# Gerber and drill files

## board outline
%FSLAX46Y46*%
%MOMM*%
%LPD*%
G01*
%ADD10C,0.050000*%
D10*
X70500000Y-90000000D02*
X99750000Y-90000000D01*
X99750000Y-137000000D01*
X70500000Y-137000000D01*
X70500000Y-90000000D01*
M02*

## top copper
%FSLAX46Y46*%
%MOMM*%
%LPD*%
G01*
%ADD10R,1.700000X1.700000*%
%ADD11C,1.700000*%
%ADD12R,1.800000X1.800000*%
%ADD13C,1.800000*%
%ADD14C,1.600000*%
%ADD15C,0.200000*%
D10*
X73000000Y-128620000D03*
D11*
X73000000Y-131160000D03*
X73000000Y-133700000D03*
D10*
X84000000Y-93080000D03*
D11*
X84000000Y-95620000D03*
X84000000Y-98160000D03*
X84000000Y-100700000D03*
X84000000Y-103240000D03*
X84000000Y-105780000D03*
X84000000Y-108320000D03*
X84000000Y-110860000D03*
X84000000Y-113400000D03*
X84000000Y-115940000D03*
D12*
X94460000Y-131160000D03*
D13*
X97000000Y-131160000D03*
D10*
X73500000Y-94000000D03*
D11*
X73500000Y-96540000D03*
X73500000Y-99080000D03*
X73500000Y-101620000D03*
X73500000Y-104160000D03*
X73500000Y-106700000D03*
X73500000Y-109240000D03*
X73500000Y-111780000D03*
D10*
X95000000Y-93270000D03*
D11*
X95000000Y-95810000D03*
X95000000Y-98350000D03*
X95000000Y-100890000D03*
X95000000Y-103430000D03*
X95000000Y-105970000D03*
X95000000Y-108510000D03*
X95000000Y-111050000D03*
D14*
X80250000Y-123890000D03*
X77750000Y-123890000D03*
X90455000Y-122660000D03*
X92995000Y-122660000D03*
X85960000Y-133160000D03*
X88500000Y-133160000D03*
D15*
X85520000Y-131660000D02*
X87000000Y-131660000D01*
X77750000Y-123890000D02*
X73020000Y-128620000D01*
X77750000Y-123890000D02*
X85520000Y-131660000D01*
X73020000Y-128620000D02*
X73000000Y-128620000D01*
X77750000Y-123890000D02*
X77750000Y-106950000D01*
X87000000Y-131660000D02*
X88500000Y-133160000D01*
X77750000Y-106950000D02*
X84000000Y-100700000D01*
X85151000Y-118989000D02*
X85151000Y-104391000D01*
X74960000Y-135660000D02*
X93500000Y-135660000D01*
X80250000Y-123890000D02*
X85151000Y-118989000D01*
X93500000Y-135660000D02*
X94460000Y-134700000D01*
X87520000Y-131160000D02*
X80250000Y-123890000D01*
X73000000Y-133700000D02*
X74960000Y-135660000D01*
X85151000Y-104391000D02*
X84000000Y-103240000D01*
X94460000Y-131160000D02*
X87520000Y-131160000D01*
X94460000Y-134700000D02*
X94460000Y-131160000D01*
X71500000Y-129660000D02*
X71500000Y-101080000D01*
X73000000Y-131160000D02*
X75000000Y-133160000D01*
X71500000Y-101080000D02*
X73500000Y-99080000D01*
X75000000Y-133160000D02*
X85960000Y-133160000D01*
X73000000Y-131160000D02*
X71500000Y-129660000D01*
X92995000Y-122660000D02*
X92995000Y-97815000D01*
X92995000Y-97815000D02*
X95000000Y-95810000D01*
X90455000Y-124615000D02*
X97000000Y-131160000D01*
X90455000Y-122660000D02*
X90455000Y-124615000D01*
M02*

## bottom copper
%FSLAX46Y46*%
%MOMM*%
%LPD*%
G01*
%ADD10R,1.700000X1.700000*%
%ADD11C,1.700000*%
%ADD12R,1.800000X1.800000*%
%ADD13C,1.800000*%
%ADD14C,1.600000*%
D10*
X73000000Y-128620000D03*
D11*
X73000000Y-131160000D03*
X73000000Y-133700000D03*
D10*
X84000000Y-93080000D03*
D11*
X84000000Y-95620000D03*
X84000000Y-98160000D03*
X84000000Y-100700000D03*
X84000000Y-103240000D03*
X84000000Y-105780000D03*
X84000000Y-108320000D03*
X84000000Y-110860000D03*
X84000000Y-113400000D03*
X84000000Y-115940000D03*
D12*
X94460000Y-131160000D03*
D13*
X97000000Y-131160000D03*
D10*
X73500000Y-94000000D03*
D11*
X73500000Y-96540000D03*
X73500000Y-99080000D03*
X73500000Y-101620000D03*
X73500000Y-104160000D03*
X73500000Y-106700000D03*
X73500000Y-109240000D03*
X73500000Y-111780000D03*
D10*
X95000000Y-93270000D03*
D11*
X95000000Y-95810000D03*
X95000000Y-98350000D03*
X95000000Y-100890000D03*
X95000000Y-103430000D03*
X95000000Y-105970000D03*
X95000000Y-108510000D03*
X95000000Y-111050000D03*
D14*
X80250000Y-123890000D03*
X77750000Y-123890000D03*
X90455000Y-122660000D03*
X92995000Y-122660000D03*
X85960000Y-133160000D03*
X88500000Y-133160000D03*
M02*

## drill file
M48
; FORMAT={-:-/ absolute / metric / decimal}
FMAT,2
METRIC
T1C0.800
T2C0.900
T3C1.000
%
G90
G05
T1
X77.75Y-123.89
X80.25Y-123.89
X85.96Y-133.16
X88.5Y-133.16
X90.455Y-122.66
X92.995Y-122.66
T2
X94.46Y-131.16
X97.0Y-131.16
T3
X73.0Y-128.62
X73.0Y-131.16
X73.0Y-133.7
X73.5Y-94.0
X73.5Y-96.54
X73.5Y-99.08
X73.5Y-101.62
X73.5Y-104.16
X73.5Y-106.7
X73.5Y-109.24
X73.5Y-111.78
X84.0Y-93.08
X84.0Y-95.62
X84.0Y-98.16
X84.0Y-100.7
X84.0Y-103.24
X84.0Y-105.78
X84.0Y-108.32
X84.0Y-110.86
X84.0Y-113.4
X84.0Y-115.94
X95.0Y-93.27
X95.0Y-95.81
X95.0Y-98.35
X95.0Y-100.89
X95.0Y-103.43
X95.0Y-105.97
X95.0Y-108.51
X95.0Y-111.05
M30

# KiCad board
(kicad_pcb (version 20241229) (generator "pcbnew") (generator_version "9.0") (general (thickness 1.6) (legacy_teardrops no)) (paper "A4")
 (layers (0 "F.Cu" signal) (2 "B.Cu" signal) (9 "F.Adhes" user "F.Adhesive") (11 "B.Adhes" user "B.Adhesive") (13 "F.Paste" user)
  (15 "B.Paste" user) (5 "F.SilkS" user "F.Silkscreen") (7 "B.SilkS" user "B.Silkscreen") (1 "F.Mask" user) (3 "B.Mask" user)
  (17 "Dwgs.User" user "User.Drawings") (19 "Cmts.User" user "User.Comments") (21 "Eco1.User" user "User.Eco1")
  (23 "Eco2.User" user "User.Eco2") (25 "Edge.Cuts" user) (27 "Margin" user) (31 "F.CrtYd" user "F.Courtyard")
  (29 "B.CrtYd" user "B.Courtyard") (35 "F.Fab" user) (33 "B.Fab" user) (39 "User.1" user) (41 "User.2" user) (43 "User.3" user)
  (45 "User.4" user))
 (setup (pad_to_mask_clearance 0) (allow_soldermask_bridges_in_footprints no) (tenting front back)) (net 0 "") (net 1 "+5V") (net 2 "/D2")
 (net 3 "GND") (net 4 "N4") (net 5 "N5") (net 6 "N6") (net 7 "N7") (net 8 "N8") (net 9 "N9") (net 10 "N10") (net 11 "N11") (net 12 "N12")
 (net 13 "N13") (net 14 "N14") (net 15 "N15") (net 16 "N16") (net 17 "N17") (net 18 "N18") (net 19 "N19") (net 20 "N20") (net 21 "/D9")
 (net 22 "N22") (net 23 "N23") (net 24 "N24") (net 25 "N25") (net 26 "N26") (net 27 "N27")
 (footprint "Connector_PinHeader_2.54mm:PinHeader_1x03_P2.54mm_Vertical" (layer "F.Cu") (at 73 128.62)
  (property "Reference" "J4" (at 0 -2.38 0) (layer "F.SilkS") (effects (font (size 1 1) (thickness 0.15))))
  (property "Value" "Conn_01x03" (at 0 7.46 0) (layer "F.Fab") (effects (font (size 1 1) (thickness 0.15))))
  (pad "1" thru_hole rect (at 0 0) (size 1.7 1.7) (drill 1) (layers "*.Cu" "*.Mask") (remove_unused_layers no) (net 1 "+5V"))
  (pad "2" thru_hole circle (at 0 2.54) (size 1.7 1.7) (drill 1) (layers "*.Cu" "*.Mask") (remove_unused_layers no) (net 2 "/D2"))
  (pad "3" thru_hole circle (at 0 5.08) (size 1.7 1.7) (drill 1) (layers "*.Cu" "*.Mask") (remove_unused_layers no) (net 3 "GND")))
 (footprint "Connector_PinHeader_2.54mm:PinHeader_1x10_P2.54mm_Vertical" (layer "F.Cu") (at 84 93.08)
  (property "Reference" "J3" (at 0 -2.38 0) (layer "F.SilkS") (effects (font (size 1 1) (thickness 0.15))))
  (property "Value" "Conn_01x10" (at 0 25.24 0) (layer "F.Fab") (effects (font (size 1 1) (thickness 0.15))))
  (pad "1" thru_hole rect (at 0 0) (size 1.7 1.7) (drill 1) (layers "*.Cu" "*.Mask") (remove_unused_layers no) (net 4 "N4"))
  (pad "2" thru_hole circle (at 0 2.54) (size 1.7 1.7) (drill 1) (layers "*.Cu" "*.Mask") (remove_unused_layers no) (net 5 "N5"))
  (pad "3" thru_hole circle (at 0 5.08) (size 1.7 1.7) (drill 1) (layers "*.Cu" "*.Mask") (remove_unused_layers no) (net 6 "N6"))
  (pad "4" thru_hole circle (at 0 7.62) (size 1.7 1.7) (drill 1) (layers "*.Cu" "*.Mask") (remove_unused_layers no) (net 1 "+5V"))
  (pad "5" thru_hole circle (at 0 10.16) (size 1.7 1.7) (drill 1) (layers "*.Cu" "*.Mask") (remove_unused_layers no) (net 3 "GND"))
  (pad "6" thru_hole circle (at 0 12.7) (size 1.7 1.7) (drill 1) (layers "*.Cu" "*.Mask") (remove_unused_layers no) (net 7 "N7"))
  (pad "7" thru_hole circle (at 0 15.24) (size 1.7 1.7) (drill 1) (layers "*.Cu" "*.Mask") (remove_unused_layers no) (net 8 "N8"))
  (pad "8" thru_hole circle (at 0 17.78) (size 1.7 1.7) (drill 1) (layers "*.Cu" "*.Mask") (remove_unused_layers no) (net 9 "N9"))
  (pad "9" thru_hole circle (at 0 20.32) (size 1.7 1.7) (drill 1) (layers "*.Cu" "*.Mask") (remove_unused_layers no) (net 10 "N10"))
  (pad "10" thru_hole circle (at 0 22.86) (size 1.7 1.7) (drill 1) (layers "*.Cu" "*.Mask") (remove_unused_layers no) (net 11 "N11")))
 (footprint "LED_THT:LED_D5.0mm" (layer "F.Cu") (at 94.46 131.16)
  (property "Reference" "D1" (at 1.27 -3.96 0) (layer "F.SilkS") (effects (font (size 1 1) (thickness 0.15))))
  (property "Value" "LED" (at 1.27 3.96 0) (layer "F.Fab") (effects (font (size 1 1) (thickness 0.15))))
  (pad "1" thru_hole rect (at 0 0) (size 1.8 1.8) (drill 0.9) (layers "*.Cu" "*.Mask") (remove_unused_layers no) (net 3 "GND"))
  (pad "2" thru_hole circle (at 2.54 0) (size 1.8 1.8) (drill 0.9) (layers "*.Cu" "*.Mask") (remove_unused_layers no) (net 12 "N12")))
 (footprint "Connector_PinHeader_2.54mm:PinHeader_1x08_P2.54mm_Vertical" (layer "F.Cu") (at 73.5 94)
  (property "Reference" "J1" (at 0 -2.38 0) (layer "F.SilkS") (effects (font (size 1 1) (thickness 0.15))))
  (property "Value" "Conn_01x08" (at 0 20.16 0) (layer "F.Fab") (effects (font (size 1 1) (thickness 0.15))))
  (pad "1" thru_hole rect (at 0 0) (size 1.7 1.7) (drill 1) (layers "*.Cu" "*.Mask") (remove_unused_layers no) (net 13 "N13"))
  (pad "2" thru_hole circle (at 0 2.54) (size 1.7 1.7) (drill 1) (layers "*.Cu" "*.Mask") (remove_unused_layers no) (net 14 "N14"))
  (pad "3" thru_hole circle (at 0 5.08) (size 1.7 1.7) (drill 1) (layers "*.Cu" "*.Mask") (remove_unused_layers no) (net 2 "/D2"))
  (pad "4" thru_hole circle (at 0 7.62) (size 1.7 1.7) (drill 1) (layers "*.Cu" "*.Mask") (remove_unused_layers no) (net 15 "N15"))
  (pad "5" thru_hole circle (at 0 10.16) (size 1.7 1.7) (drill 1) (layers "*.Cu" "*.Mask") (remove_unused_layers no) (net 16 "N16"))
  (pad "6" thru_hole circle (at 0 12.7) (size 1.7 1.7) (drill 1) (layers "*.Cu" "*.Mask") (remove_unused_layers no) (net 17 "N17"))
  (pad "7" thru_hole circle (at 0 15.24) (size 1.7 1.7) (drill 1) (layers "*.Cu" "*.Mask") (remove_unused_layers no) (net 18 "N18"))
  (pad "8" thru_hole circle (at 0 17.78) (size 1.7 1.7) (drill 1) (layers "*.Cu" "*.Mask") (remove_unused_layers no) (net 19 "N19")))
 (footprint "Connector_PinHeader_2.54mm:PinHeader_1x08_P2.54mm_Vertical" (layer "F.Cu") (at 95 93.27)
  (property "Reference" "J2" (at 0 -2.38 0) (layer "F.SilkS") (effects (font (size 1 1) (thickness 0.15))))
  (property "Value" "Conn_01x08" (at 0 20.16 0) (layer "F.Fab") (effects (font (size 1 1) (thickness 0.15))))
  (pad "1" thru_hole rect (at 0 0) (size 1.7 1.7) (drill 1) (layers "*.Cu" "*.Mask") (remove_unused_layers no) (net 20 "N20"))
  (pad "2" thru_hole circle (at 0 2.54) (size 1.7 1.7) (drill 1) (layers "*.Cu" "*.Mask") (remove_unused_layers no) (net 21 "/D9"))
  (pad "3" thru_hole circle (at 0 5.08) (size 1.7 1.7) (drill 1) (layers "*.Cu" "*.Mask") (remove_unused_layers no) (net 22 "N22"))
  (pad "4" thru_hole circle (at 0 7.62) (size 1.7 1.7) (drill 1) (layers "*.Cu" "*.Mask") (remove_unused_layers no) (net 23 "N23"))
  (pad "5" thru_hole circle (at 0 10.16) (size 1.7 1.7) (drill 1) (layers "*.Cu" "*.Mask") (remove_unused_layers no) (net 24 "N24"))
  (pad "6" thru_hole circle (at 0 12.7) (size 1.7 1.7) (drill 1) (layers "*.Cu" "*.Mask") (remove_unused_layers no) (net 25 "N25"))
  (pad "7" thru_hole circle (at 0 15.24) (size 1.7 1.7) (drill 1) (layers "*.Cu" "*.Mask") (remove_unused_layers no) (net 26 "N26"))
  (pad "8" thru_hole circle (at 0 17.78) (size 1.7 1.7) (drill 1) (layers "*.Cu" "*.Mask") (remove_unused_layers no) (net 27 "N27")))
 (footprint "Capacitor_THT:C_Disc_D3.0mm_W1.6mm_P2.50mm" (layer "F.Cu") (at 80.25 123.89 180)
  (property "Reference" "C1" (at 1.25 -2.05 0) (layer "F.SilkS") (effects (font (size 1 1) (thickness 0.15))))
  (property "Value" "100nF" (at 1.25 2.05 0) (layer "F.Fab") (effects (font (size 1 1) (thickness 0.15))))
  (pad "1" thru_hole circle (at 0 0 180) (size 1.6 1.6) (drill 0.8) (layers "*.Cu" "*.Mask") (remove_unused_layers no) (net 3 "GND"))
  (pad "2" thru_hole circle (at 2.5 0 180) (size 1.6 1.6) (drill 0.8) (layers "*.Cu" "*.Mask") (remove_unused_layers no) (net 1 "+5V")))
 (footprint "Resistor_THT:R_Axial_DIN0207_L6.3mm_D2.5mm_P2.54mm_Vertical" (layer "F.Cu") (at 90.455 122.66)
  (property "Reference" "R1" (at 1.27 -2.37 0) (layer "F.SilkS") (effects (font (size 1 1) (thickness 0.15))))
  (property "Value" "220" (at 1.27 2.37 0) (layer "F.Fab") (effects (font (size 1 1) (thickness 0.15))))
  (pad "1" thru_hole circle (at 0 0) (size 1.6 1.6) (drill 0.8) (layers "*.Cu" "*.Mask") (remove_unused_layers no) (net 12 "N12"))
  (pad "2" thru_hole circle (at 2.54 0) (size 1.6 1.6) (drill 0.8) (layers "*.Cu" "*.Mask") (remove_unused_layers no) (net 21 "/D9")))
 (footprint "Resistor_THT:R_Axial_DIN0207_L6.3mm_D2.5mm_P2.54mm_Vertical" (layer "F.Cu") (at 85.96 133.16)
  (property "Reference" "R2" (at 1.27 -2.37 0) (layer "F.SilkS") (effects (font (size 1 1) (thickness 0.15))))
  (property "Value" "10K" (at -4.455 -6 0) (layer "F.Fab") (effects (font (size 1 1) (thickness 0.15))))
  (pad "1" thru_hole circle (at 0 0) (size 1.6 1.6) (drill 0.8) (layers "*.Cu" "*.Mask") (remove_unused_layers no) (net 2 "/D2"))
  (pad "2" thru_hole circle (at 2.54 0) (size 1.6 1.6) (drill 0.8) (layers "*.Cu" "*.Mask") (remove_unused_layers no) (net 1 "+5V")))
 (gr_rect (start 70.5 90) (end 99.75 137) (stroke (width 0.05) (type default)) (fill no) (layer "Edge.Cuts"))
 (segment (start 85.52 131.66) (end 87 131.66) (width 0.2) (layer "F.Cu") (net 1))
 (segment (start 77.75 123.89) (end 73.02 128.62) (width 0.2) (layer "F.Cu") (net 1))
 (segment (start 77.75 123.89) (end 85.52 131.66) (width 0.2) (layer "F.Cu") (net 1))
 (segment (start 73.02 128.62) (end 73 128.62) (width 0.2) (layer "F.Cu") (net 1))
 (segment (start 77.75 123.89) (end 77.75 106.95) (width 0.2) (layer "F.Cu") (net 1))
 (segment (start 87 131.66) (end 88.5 133.16) (width 0.2) (layer "F.Cu") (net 1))
 (segment (start 77.75 106.95) (end 84 100.7) (width 0.2) (layer "F.Cu") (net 1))
 (segment (start 85.151 118.989) (end 85.151 104.391) (width 0.2) (layer "F.Cu") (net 3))
 (segment (start 74.96 135.66) (end 93.5 135.66) (width 0.2) (layer "F.Cu") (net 3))
 (segment (start 80.25 123.89) (end 85.151 118.989) (width 0.2) (layer "F.Cu") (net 3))
 (segment (start 93.5 135.66) (end 94.46 134.7) (width 0.2) (layer "F.Cu") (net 3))
 (segment (start 87.52 131.16) (end 80.25 123.89) (width 0.2) (layer "F.Cu") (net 3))
 (segment (start 73 133.7) (end 74.96 135.66) (width 0.2) (layer "F.Cu") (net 3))
 (segment (start 85.151 104.391) (end 84 103.24) (width 0.2) (layer "F.Cu") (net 3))
 (segment (start 94.46 131.16) (end 87.52 131.16) (width 0.2) (layer "F.Cu") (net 3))
 (segment (start 94.46 134.7) (end 94.46 131.16) (width 0.2) (layer "F.Cu") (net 3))
 (segment (start 71.5 129.66) (end 71.5 101.08) (width 0.2) (layer "F.Cu") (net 2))
 (segment (start 73 131.16) (end 75 133.16) (width 0.2) (layer "F.Cu") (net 2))
 (segment (start 71.5 101.08) (end 73.5 99.08) (width 0.2) (layer "F.Cu") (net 2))
 (segment (start 75 133.16) (end 85.96 133.16) (width 0.2) (layer "F.Cu") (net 2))
 (segment (start 73 131.16) (end 71.5 129.66) (width 0.2) (layer "F.Cu") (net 2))
 (segment (start 92.995 122.66) (end 92.995 97.815) (width 0.2) (layer "F.Cu") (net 21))
 (segment (start 92.995 97.815) (end 95 95.81) (width 0.2) (layer "F.Cu") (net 21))
 (segment (start 90.455 124.615) (end 97 131.16) (width 0.2) (layer "F.Cu") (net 12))
 (segment (start 90.455 122.66) (end 90.455 124.615) (width 0.2) (layer "F.Cu") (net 12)))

